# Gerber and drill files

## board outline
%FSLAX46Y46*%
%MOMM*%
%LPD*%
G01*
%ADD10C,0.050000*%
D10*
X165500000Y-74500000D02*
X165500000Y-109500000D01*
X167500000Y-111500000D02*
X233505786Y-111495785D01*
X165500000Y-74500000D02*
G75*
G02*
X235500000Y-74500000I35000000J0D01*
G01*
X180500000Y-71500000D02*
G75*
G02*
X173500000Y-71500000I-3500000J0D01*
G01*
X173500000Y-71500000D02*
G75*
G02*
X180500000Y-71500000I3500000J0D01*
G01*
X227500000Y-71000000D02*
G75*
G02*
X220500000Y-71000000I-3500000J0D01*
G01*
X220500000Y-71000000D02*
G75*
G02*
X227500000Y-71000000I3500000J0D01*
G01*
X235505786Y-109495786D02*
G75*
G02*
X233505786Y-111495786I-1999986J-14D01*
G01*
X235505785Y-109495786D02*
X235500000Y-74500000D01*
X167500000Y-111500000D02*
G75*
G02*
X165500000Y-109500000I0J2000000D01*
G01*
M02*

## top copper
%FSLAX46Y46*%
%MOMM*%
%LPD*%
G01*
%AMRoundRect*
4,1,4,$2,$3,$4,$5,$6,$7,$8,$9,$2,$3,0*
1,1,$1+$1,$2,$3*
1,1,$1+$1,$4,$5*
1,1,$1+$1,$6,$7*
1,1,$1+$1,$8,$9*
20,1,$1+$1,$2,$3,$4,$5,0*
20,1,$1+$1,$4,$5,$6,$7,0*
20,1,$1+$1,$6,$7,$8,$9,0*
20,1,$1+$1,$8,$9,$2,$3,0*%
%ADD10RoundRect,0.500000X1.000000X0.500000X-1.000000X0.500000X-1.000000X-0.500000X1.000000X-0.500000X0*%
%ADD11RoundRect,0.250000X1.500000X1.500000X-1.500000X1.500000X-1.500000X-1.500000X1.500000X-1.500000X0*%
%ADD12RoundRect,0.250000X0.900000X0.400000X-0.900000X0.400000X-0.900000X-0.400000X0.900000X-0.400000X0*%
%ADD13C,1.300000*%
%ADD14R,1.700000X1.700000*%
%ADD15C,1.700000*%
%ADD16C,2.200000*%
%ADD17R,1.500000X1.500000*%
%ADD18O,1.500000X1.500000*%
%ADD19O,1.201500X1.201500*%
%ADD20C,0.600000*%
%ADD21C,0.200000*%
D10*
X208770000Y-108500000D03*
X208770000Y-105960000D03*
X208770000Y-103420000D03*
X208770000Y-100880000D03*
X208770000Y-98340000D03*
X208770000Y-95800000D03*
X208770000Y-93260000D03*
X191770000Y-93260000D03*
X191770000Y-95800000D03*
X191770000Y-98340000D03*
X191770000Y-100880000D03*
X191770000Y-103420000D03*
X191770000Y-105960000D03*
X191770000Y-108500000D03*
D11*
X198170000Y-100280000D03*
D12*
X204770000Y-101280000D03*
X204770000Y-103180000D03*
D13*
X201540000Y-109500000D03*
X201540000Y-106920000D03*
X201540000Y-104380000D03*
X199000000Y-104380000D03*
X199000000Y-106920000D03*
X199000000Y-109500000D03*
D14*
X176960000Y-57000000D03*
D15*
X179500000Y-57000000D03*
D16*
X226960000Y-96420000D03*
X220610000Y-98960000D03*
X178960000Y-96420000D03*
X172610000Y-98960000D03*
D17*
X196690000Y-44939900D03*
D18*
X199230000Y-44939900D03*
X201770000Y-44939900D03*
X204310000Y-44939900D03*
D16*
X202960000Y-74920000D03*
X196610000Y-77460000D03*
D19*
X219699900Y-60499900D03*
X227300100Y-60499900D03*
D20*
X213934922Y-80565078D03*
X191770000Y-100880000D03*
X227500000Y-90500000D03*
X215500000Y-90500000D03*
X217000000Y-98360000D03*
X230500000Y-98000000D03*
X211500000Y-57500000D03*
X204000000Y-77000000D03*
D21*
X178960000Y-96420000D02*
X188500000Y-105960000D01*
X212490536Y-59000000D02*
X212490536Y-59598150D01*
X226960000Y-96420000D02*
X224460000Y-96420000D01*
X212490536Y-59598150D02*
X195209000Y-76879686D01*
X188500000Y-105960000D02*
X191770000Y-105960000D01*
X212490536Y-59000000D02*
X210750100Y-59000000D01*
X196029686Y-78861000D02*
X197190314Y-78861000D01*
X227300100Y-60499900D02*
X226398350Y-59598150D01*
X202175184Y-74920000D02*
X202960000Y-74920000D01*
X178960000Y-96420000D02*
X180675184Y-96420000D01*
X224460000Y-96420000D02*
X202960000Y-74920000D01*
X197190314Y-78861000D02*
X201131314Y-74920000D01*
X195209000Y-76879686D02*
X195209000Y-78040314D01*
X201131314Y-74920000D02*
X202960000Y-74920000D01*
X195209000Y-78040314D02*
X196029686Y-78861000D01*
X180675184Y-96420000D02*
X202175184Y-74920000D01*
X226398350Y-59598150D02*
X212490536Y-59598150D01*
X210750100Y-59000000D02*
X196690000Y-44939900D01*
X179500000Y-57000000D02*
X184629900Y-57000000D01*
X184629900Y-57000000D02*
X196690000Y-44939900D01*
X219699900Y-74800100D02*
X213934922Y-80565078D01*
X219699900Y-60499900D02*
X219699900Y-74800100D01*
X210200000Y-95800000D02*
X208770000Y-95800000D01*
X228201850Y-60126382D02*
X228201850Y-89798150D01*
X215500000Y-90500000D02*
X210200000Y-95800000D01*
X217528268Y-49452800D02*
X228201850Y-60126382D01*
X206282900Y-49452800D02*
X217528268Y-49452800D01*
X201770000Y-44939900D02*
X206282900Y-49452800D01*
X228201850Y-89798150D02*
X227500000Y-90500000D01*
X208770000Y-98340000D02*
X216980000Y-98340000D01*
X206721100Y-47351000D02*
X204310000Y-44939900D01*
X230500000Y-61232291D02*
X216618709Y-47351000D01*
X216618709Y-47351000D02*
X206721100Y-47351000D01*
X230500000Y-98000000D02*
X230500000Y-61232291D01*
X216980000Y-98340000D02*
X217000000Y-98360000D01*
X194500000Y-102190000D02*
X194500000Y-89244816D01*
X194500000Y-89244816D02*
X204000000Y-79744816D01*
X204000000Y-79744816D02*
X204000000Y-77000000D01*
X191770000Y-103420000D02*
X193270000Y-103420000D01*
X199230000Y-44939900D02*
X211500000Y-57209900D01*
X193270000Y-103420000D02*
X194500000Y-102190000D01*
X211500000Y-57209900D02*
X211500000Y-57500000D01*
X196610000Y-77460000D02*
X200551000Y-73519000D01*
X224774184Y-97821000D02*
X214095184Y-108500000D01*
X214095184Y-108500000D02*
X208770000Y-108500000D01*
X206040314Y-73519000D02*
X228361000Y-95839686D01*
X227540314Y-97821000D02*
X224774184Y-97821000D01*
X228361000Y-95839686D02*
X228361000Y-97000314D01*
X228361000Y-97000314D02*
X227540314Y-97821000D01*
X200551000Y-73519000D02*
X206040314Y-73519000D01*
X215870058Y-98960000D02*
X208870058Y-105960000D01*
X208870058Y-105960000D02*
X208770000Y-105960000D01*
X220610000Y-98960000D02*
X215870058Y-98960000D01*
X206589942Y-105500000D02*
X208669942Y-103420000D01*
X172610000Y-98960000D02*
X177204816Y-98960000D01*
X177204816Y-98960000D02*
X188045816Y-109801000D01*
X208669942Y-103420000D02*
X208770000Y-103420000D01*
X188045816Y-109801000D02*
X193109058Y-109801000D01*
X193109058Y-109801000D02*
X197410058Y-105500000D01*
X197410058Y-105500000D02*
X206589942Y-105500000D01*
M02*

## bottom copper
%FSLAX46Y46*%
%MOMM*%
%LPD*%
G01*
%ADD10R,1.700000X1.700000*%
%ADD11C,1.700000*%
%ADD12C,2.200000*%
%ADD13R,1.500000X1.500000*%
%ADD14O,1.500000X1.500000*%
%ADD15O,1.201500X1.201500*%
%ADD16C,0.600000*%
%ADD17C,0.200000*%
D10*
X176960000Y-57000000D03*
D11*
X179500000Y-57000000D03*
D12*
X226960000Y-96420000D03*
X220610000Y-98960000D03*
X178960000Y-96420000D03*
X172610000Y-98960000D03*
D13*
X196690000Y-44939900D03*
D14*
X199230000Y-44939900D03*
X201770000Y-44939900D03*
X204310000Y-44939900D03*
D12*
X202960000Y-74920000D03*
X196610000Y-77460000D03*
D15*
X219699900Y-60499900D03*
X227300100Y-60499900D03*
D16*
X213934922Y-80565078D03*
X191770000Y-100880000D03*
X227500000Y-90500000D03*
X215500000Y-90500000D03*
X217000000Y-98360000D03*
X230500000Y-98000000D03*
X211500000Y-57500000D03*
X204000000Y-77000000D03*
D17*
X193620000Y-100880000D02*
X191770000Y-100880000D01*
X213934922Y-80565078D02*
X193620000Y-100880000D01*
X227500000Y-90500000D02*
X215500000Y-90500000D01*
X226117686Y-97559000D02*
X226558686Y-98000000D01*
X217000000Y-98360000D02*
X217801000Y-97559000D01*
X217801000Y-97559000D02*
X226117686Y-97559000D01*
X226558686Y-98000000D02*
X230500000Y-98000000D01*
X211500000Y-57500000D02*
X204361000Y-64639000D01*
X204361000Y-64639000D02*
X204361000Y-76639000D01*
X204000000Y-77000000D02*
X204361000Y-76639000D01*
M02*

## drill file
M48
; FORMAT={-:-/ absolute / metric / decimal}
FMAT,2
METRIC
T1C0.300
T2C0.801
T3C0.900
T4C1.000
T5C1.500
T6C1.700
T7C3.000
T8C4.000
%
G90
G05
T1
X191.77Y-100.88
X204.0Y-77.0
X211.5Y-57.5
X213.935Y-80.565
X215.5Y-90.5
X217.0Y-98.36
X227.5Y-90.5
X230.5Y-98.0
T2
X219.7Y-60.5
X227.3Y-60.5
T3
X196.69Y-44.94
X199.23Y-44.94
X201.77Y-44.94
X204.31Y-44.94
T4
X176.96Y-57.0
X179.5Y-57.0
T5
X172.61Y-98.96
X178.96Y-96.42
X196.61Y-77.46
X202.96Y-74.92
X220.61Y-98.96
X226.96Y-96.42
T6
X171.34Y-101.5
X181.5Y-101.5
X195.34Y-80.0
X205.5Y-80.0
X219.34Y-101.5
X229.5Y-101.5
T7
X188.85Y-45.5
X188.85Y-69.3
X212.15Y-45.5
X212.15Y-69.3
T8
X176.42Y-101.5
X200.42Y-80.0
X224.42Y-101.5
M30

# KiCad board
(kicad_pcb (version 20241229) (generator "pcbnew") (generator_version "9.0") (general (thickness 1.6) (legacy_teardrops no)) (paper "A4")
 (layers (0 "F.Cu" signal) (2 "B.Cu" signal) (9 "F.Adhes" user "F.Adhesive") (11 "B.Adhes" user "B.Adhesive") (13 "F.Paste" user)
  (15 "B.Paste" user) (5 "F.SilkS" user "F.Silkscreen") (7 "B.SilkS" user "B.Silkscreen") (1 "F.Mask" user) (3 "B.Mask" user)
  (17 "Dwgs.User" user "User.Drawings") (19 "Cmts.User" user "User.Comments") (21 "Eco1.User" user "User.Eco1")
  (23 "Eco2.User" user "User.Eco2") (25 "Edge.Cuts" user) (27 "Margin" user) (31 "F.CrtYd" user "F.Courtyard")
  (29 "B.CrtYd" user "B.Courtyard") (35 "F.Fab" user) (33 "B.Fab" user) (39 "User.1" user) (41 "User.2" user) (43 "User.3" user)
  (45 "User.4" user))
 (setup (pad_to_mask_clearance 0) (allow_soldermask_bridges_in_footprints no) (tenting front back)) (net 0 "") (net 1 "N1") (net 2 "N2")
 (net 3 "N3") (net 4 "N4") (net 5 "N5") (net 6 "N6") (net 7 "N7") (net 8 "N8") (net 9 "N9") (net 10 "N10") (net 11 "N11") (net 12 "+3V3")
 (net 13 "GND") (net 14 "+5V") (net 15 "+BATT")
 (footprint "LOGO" (layer "F.Cu") (at 225.5 79.5 -90)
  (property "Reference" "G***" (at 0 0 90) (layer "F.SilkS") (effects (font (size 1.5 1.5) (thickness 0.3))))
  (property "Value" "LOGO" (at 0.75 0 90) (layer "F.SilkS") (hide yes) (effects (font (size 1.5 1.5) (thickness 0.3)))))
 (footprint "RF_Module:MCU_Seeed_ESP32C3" (layer "F.Cu") (at 200.27 100.88 180)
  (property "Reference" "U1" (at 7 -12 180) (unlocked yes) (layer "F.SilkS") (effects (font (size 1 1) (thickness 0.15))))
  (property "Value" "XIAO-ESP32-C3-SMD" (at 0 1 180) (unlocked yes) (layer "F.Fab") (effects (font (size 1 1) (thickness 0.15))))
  (pad "" smd roundrect (at 1.1 -0.4 180) (size 1.5 1.5) (layers "F.Paste") (roundrect_rratio 0.1666666667))
  (pad "" smd roundrect (at 1.1 1.6 180) (size 1.5 1.5) (layers "F.Paste") (roundrect_rratio 0.1666666667))
  (pad "" smd roundrect (at 3.1 -0.4 180) (size 1.5 1.5) (layers "F.Paste") (roundrect_rratio 0.1666666667))
  (pad "" smd roundrect (at 3.1 1.6 180) (size 1.5 1.5) (layers "F.Paste") (roundrect_rratio 0.1666666667))
  (pad "1" smd roundrect (at -8.5 -7.62 180) (size 3 2) (layers "F.Cu" "F.Mask" "F.Paste") (roundrect_rratio 0.25) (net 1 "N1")
   (thermal_bridge_angle 45))
  (pad "2" smd roundrect (at -8.5 -5.08 180) (size 3 2) (layers "F.Cu" "F.Mask" "F.Paste") (roundrect_rratio 0.25) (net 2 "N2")
   (thermal_bridge_angle 45))
  (pad "3" smd roundrect (at -8.5 -2.54 180) (size 3 2) (layers "F.Cu" "F.Mask" "F.Paste") (roundrect_rratio 0.25) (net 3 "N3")
   (thermal_bridge_angle 45))
  (pad "4" smd roundrect (at -8.5 0 180) (size 3 2) (layers "F.Cu" "F.Mask" "F.Paste") (roundrect_rratio 0.25) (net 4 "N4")
   (thermal_bridge_angle 45))
  (pad "5" smd roundrect (at -8.5 2.54 180) (size 3 2) (layers "F.Cu" "F.Mask" "F.Paste") (roundrect_rratio 0.25) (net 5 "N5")
   (thermal_bridge_angle 45))
  (pad "6" smd roundrect (at -8.5 5.08 180) (size 3 2) (layers "F.Cu" "F.Mask" "F.Paste") (roundrect_rratio 0.25) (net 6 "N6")
   (thermal_bridge_angle 45))
  (pad "7" smd roundrect (at -8.5 7.62 180) (size 3 2) (layers "F.Cu" "F.Mask" "F.Paste") (roundrect_rratio 0.25) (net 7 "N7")
   (thermal_bridge_angle 45))
  (pad "8" smd roundrect (at 8.5 7.62 180) (size 3 2) (layers "F.Cu" "F.Mask" "F.Paste") (roundrect_rratio 0.25) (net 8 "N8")
   (thermal_bridge_angle 45))
  (pad "9" smd roundrect (at 8.5 5.08 180) (size 3 2) (layers "F.Cu" "F.Mask" "F.Paste") (roundrect_rratio 0.25) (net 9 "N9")
   (thermal_bridge_angle 45))
  (pad "10" smd roundrect (at 8.5 2.54 180) (size 3 2) (layers "F.Cu" "F.Mask" "F.Paste") (roundrect_rratio 0.25) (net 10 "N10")
   (thermal_bridge_angle 45))
  (pad "11" smd roundrect (at 8.5 0 180) (size 3 2) (layers "F.Cu" "F.Mask" "F.Paste") (roundrect_rratio 0.25) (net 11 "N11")
   (thermal_bridge_angle 45))
  (pad "12" smd roundrect (at 8.5 -2.54 180) (size 3 2) (layers "F.Cu" "F.Mask" "F.Paste") (roundrect_rratio 0.25) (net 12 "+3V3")
   (thermal_bridge_angle 45))
  (pad "13" smd roundrect (at 8.5 -5.08 180) (size 3 2) (layers "F.Cu" "F.Mask" "F.Paste") (roundrect_rratio 0.25) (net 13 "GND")
   (thermal_bridge_angle 45))
  (pad "14" smd roundrect (at 8.5 -7.62 180) (size 3 2) (layers "F.Cu" "F.Mask" "F.Paste") (roundrect_rratio 0.25) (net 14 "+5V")
   (thermal_bridge_angle 45))
  (pad "15" smd roundrect (at 2.1 0.6 180) (size 3.5 3.5) (layers "F.Cu" "F.Mask") (roundrect_rratio 0.07142857143))
  (pad "16" smd roundrect (at -4.5 -0.4 180) (size 2.3 1.3) (layers "F.Cu" "F.Mask" "F.Paste") (roundrect_rratio 0.1923076923))
  (pad "17" smd roundrect (at -4.5 -2.3 180) (size 2.3 1.3) (layers "F.Cu" "F.Mask" "F.Paste") (roundrect_rratio 0.1923076923))
  (pad "18" smd circle (at -1.27 -8.62 180) (size 1.3 1.3) (layers "F.Cu" "F.Mask" "F.Paste"))
  (pad "19" smd circle (at -1.27 -6.04 180) (size 1.3 1.3) (layers "F.Cu" "F.Mask" "F.Paste"))
  (pad "20" smd circle (at -1.27 -3.5 180) (size 1.3 1.3) (layers "F.Cu" "F.Mask" "F.Paste"))
  (pad "21" smd circle (at 1.27 -3.5 180) (size 1.3 1.3) (layers "F.Cu" "F.Mask" "F.Paste"))
  (pad "22" smd circle (at 1.27 -6.04 180) (size 1.3 1.3) (layers "F.Cu" "F.Mask" "F.Paste"))
  (pad "23" smd circle (at 1.27 -8.62 180) (size 1.3 1.3) (layers "F.Cu" "F.Mask" "F.Paste")))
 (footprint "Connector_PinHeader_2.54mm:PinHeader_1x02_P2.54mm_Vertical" (layer "F.Cu") (at 176.96 57 90)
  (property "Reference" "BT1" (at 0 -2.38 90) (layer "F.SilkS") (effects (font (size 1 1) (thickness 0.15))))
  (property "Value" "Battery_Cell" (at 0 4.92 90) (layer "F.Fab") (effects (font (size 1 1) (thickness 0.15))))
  (pad "1" thru_hole rect (at 0 0 90) (size 1.7 1.7) (drill 1) (layers "*.Cu" "*.Mask") (remove_unused_layers no) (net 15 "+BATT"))
  (pad "2" thru_hole circle (at 0 2.54 90) (size 1.7 1.7) (drill 1) (layers "*.Cu" "*.Mask") (remove_unused_layers no) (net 13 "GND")))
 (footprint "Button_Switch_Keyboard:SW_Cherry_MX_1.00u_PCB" (layer "F.Cu") (at 226.96 96.42)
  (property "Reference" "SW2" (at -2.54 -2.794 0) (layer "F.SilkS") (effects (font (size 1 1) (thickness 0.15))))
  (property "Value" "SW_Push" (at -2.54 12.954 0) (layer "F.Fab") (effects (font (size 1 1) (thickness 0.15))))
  (pad "" np_thru_hole circle (at -7.62 5.08) (size 1.7 1.7) (drill 1.7) (layers "*.Cu" "*.Mask"))
  (pad "" np_thru_hole circle (at -2.54 5.08) (size 4 4) (drill 4) (layers "*.Cu" "*.Mask"))
  (pad "" np_thru_hole circle (at 2.54 5.08) (size 1.7 1.7) (drill 1.7) (layers "*.Cu" "*.Mask"))
  (pad "1" thru_hole circle (at 0 0) (size 2.2 2.2) (drill 1.5) (layers "*.Cu" "*.Mask") (remove_unused_layers no) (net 13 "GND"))
  (pad "2" thru_hole circle (at -6.35 2.54) (size 2.2 2.2) (drill 1.5) (layers "*.Cu" "*.Mask") (remove_unused_layers no) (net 2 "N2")))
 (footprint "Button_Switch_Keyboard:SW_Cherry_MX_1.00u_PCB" (layer "F.Cu") (at 178.96 96.42)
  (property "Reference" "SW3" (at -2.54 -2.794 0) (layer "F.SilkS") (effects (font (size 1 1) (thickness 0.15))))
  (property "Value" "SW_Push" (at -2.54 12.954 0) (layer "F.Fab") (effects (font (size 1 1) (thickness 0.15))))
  (pad "" np_thru_hole circle (at -7.62 5.08) (size 1.7 1.7) (drill 1.7) (layers "*.Cu" "*.Mask"))
  (pad "" np_thru_hole circle (at -2.54 5.08) (size 4 4) (drill 4) (layers "*.Cu" "*.Mask"))
  (pad "" np_thru_hole circle (at 2.54 5.08) (size 1.7 1.7) (drill 1.7) (layers "*.Cu" "*.Mask"))
  (pad "1" thru_hole circle (at 0 0) (size 2.2 2.2) (drill 1.5) (layers "*.Cu" "*.Mask") (remove_unused_layers no) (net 13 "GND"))
  (pad "2" thru_hole circle (at -6.35 2.54) (size 2.2 2.2) (drill 1.5) (layers "*.Cu" "*.Mask") (remove_unused_layers no) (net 3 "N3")))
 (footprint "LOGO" (layer "F.Cu") (at 177.5 78)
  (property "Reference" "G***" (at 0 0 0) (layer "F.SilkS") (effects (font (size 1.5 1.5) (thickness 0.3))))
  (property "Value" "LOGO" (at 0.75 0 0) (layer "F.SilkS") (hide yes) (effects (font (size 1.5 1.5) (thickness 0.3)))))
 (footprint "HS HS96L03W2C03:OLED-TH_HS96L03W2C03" (layer "F.Cu") (at 200.5 44.9399)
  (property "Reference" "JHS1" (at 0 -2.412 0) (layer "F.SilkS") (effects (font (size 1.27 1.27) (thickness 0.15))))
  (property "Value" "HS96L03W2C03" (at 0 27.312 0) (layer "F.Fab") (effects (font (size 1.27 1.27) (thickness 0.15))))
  (pad "" np_thru_hole circle (at -11.65 0.5601) (size 3 3) (drill 3) (layers "*.Cu" "*.Mask"))
  (pad "" np_thru_hole circle (at -11.65 24.3599) (size 3 3) (drill 3) (layers "*.Cu" "*.Mask"))
  (pad "" np_thru_hole circle (at 11.65 0.5601) (size 3 3) (drill 3) (layers "*.Cu" "*.Mask"))
  (pad "" np_thru_hole circle (at 11.65 24.3599) (size 3 3) (drill 3) (layers "*.Cu" "*.Mask"))
  (pad "1" thru_hole rect (at -3.81 0) (size 1.5 1.5) (drill 0.9) (layers "*.Cu" "*.Mask") (remove_unused_layers no) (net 13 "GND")
   (solder_mask_margin 0.05) (solder_paste_margin 0) (thermal_bridge_angle 0))
  (pad "2" thru_hole oval (at -1.27 0) (size 1.5 1.5) (drill 0.9) (layers "*.Cu" "*.Mask") (remove_unused_layers no) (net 12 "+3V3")
   (solder_mask_margin 0.05) (solder_paste_margin 0) (thermal_bridge_angle 0))
  (pad "3" thru_hole oval (at 1.27 0) (size 1.5 1.5) (drill 0.9) (layers "*.Cu" "*.Mask") (remove_unused_layers no) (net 6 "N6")
   (solder_mask_margin 0.05) (solder_paste_margin 0) (thermal_bridge_angle 0))
  (pad "4" thru_hole oval (at 3.81 0) (size 1.5 1.5) (drill 0.9) (layers "*.Cu" "*.Mask") (remove_unused_layers no) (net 5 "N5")
   (solder_mask_margin 0.05) (solder_paste_margin 0) (thermal_bridge_angle 0))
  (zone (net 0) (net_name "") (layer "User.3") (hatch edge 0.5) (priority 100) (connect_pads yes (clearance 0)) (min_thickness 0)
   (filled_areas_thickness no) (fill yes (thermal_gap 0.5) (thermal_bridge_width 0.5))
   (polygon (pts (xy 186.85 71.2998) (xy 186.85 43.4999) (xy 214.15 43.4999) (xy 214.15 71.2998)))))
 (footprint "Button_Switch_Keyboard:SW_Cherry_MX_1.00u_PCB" (layer "F.Cu") (at 202.96 74.92)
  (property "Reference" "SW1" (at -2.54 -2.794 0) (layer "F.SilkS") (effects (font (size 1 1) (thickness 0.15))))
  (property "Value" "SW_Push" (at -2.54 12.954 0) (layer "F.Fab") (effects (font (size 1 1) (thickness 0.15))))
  (pad "" np_thru_hole circle (at -7.62 5.08) (size 1.7 1.7) (drill 1.7) (layers "*.Cu" "*.Mask"))
  (pad "" np_thru_hole circle (at -2.54 5.08) (size 4 4) (drill 4) (layers "*.Cu" "*.Mask"))
  (pad "" np_thru_hole circle (at 2.54 5.08) (size 1.7 1.7) (drill 1.7) (layers "*.Cu" "*.Mask"))
  (pad "1" thru_hole circle (at 0 0) (size 2.2 2.2) (drill 1.5) (layers "*.Cu" "*.Mask") (remove_unused_layers no) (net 13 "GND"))
  (pad "2" thru_hole circle (at -6.35 2.54) (size 2.2 2.2) (drill 1.5) (layers "*.Cu" "*.Mask") (remove_unused_layers no) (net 1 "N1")))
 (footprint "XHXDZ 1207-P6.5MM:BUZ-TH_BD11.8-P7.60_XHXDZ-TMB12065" (layer "F.Cu") (at 223.5 60.5 90)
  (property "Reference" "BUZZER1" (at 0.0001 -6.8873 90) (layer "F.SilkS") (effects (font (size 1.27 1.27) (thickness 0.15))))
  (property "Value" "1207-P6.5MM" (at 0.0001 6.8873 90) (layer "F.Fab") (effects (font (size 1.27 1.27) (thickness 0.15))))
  (pad "1" thru_hole oval (at 0.0001 -3.8001) (size 1.2015 1.2015) (drill 0.801) (layers "*.Cu" "*.Mask") (remove_unused_layers no)
   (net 11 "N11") (solder_mask_margin 0.0508) (solder_paste_margin 0) (thermal_bridge_angle 0))
  (pad "2" thru_hole oval (at 0.0001 3.8001 180) (size 1.2015 1.2015) (drill 0.801) (layers "*.Cu" "*.Mask") (remove_unused_layers no)
   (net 13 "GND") (solder_mask_margin 0.0508) (solder_paste_margin 0) (thermal_bridge_angle 0))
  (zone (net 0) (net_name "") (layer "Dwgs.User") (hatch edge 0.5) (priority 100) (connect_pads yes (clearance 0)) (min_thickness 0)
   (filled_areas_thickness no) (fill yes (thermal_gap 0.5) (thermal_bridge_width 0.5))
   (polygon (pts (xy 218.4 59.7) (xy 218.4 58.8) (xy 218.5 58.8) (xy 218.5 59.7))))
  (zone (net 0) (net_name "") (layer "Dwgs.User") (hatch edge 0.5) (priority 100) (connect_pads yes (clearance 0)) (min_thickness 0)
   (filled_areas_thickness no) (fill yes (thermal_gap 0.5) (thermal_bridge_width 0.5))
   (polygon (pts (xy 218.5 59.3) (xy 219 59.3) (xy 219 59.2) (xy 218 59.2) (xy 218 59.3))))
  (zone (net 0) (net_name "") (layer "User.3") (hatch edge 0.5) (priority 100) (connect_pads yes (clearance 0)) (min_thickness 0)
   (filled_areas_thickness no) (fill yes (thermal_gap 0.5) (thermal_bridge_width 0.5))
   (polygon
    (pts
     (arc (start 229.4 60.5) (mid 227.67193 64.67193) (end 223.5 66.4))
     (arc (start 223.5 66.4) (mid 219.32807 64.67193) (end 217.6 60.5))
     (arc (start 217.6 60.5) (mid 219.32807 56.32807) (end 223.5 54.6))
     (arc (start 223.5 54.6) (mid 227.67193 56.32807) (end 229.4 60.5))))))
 (gr_line (start 165.5 74.5) (end 165.5 109.5) (stroke (width 0.05) (type default)) (layer "Edge.Cuts"))
 (gr_line (start 167.5 111.5) (end 233.505786 111.495785) (stroke (width 0.05) (type default)) (layer "Edge.Cuts"))
 (gr_arc (start 165.5 74.5) (mid 200.5 39.5) (end 235.5 74.5) (stroke (width 0.05) (type default)) (layer "Edge.Cuts"))
 (gr_circle (center 177 71.5) (end 180.5 71.5) (stroke (width 0.05) (type default)) (fill no) (layer "Edge.Cuts"))
 (gr_circle (center 224 71) (end 227.5 71) (stroke (width 0.05) (type default)) (fill no) (layer "Edge.Cuts"))
 (gr_arc (start 235.505786 109.495786) (mid 234.92 110.91) (end 233.505786 111.495786) (stroke (width 0.05) (type default))
  (layer "Edge.Cuts"))
 (gr_line (start 235.505785 109.495786) (end 235.5 74.5) (stroke (width 0.05) (type default)) (layer "Edge.Cuts"))
 (gr_arc (start 167.5 111.5) (mid 166.085786 110.914214) (end 165.5 109.5) (stroke (width 0.05) (type default)) (layer "Edge.Cuts"))
 (segment (start 178.96 96.42) (end 188.5 105.96) (width 0.2) (layer "F.Cu") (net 13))
 (segment (start 212.490536 59) (end 212.490536 59.59815) (width 0.2) (layer "F.Cu") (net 13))
 (segment (start 226.96 96.42) (end 224.46 96.42) (width 0.2) (layer "F.Cu") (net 13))
 (segment (start 212.490536 59.59815) (end 195.209 76.879686) (width 0.2) (layer "F.Cu") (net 13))
 (segment (start 188.5 105.96) (end 191.77 105.96) (width 0.2) (layer "F.Cu") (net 13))
 (segment (start 212.490536 59) (end 210.7501 59) (width 0.2) (layer "F.Cu") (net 13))
 (segment (start 196.029686 78.861) (end 197.190314 78.861) (width 0.2) (layer "F.Cu") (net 13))
 (segment (start 227.3001 60.4999) (end 226.39835 59.59815) (width 0.2) (layer "F.Cu") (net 13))
 (segment (start 202.175184 74.92) (end 202.96 74.92) (width 0.2) (layer "F.Cu") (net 13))
 (segment (start 178.96 96.42) (end 180.675184 96.42) (width 0.2) (layer "F.Cu") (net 13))
 (segment (start 224.46 96.42) (end 202.96 74.92) (width 0.2) (layer "F.Cu") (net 13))
 (segment (start 197.190314 78.861) (end 201.131314 74.92) (width 0.2) (layer "F.Cu") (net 13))
 (segment (start 195.209 76.879686) (end 195.209 78.040314) (width 0.2) (layer "F.Cu") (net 13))
 (segment (start 201.131314 74.92) (end 202.96 74.92) (width 0.2) (layer "F.Cu") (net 13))
 (segment (start 195.209 78.040314) (end 196.029686 78.861) (width 0.2) (layer "F.Cu") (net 13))
 (segment (start 180.675184 96.42) (end 202.175184 74.92) (width 0.2) (layer "F.Cu") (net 13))
 (segment (start 226.39835 59.59815) (end 212.490536 59.59815) (width 0.2) (layer "F.Cu") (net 13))
 (segment (start 210.7501 59) (end 196.69 44.9399) (width 0.2) (layer "F.Cu") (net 13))
 (segment (start 179.5 57) (end 184.6299 57) (width 0.2) (layer "F.Cu") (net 13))
 (segment (start 184.6299 57) (end 196.69 44.9399) (width 0.2) (layer "F.Cu") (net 13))
 (segment (start 219.6999 74.8001) (end 213.934922 80.565078) (width 0.2) (layer "F.Cu") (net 11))
 (segment (start 219.6999 60.4999) (end 219.6999 74.8001) (width 0.2) (layer "F.Cu") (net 11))
 (via (at 213.934922 80.565078) (size 0.6) (drill 0.3) (layers "F.Cu" "B.Cu") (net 11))
 (via (at 191.77 100.88) (size 0.6) (drill 0.3) (layers "F.Cu" "B.Cu") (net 11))
 (segment (start 193.62 100.88) (end 191.77 100.88) (width 0.2) (layer "B.Cu") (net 11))
 (segment (start 213.934922 80.565078) (end 193.62 100.88) (width 0.2) (layer "B.Cu") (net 11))
 (segment (start 210.2 95.8) (end 208.77 95.8) (width 0.2) (layer "F.Cu") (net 6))
 (segment (start 228.20185 60.126382) (end 228.20185 89.79815) (width 0.2) (layer "F.Cu") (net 6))
 (segment (start 215.5 90.5) (end 210.2 95.8) (width 0.2) (layer "F.Cu") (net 6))
 (segment (start 217.528268 49.4528) (end 228.20185 60.126382) (width 0.2) (layer "F.Cu") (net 6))
 (segment (start 206.2829 49.4528) (end 217.528268 49.4528) (width 0.2) (layer "F.Cu") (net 6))
 (segment (start 201.77 44.9399) (end 206.2829 49.4528) (width 0.2) (layer "F.Cu") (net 6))
 (segment (start 228.20185 89.79815) (end 227.5 90.5) (width 0.2) (layer "F.Cu") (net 6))
 (via (at 227.5 90.5) (size 0.6) (drill 0.3) (layers "F.Cu" "B.Cu") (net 6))
 (via (at 215.5 90.5) (size 0.6) (drill 0.3) (layers "F.Cu" "B.Cu") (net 6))
 (segment (start 227.5 90.5) (end 215.5 90.5) (width 0.2) (layer "B.Cu") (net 6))
 (segment (start 208.77 98.34) (end 216.98 98.34) (width 0.2) (layer "F.Cu") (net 5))
 (segment (start 206.7211 47.351) (end 204.31 44.9399) (width 0.2) (layer "F.Cu") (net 5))
 (segment (start 230.5 61.232291) (end 216.618709 47.351) (width 0.2) (layer "F.Cu") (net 5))
 (segment (start 216.618709 47.351) (end 206.7211 47.351) (width 0.2) (layer "F.Cu") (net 5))
 (segment (start 230.5 98) (end 230.5 61.232291) (width 0.2) (layer "F.Cu") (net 5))
 (segment (start 216.98 98.34) (end 217 98.36) (width 0.2) (layer "F.Cu") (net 5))
 (via (at 217 98.36) (size 0.6) (drill 0.3) (layers "F.Cu" "B.Cu") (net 5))
 (via (at 230.5 98) (size 0.6) (drill 0.3) (layers "F.Cu" "B.Cu") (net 5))
 (segment (start 226.117686 97.559) (end 226.558686 98) (width 0.2) (layer "B.Cu") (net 5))
 (segment (start 217 98.36) (end 217.801 97.559) (width 0.2) (layer "B.Cu") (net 5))
 (segment (start 217.801 97.559) (end 226.117686 97.559) (width 0.2) (layer "B.Cu") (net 5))
 (segment (start 226.558686 98) (end 230.5 98) (width 0.2) (layer "B.Cu") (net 5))
 (segment (start 194.5 102.19) (end 194.5 89.244816) (width 0.2) (layer "F.Cu") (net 12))
 (segment (start 194.5 89.244816) (end 204 79.744816) (width 0.2) (layer "F.Cu") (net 12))
 (segment (start 204 79.744816) (end 204 77) (width 0.2) (layer "F.Cu") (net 12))
 (segment (start 191.77 103.42) (end 193.27 103.42) (width 0.2) (layer "F.Cu") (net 12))
 (segment (start 199.23 44.9399) (end 211.5 57.2099) (width 0.2) (layer "F.Cu") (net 12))
 (segment (start 193.27 103.42) (end 194.5 102.19) (width 0.2) (layer "F.Cu") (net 12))
 (segment (start 211.5 57.2099) (end 211.5 57.5) (width 0.2) (layer "F.Cu") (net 12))
 (via (at 211.5 57.5) (size 0.6) (drill 0.3) (layers "F.Cu" "B.Cu") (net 12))
 (via (at 204 77) (size 0.6) (drill 0.3) (layers "F.Cu" "B.Cu") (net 12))
 (segment (start 211.5 57.5) (end 204.361 64.639) (width 0.2) (layer "B.Cu") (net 12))
 (segment (start 204.361 64.639) (end 204.361 76.639) (width 0.2) (layer "B.Cu") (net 12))
 (segment (start 204 77) (end 204.361 76.639) (width 0.2) (layer "B.Cu") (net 12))
 (segment (start 196.61 77.46) (end 200.551 73.519) (width 0.2) (layer "F.Cu") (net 1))
 (segment (start 224.774184 97.821) (end 214.095184 108.5) (width 0.2) (layer "F.Cu") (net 1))
 (segment (start 214.095184 108.5) (end 208.77 108.5) (width 0.2) (layer "F.Cu") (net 1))
 (segment (start 206.040314 73.519) (end 228.361 95.839686) (width 0.2) (layer "F.Cu") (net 1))
 (segment (start 227.540314 97.821) (end 224.774184 97.821) (width 0.2) (layer "F.Cu") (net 1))
 (segment (start 228.361 95.839686) (end 228.361 97.000314) (width 0.2) (layer "F.Cu") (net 1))
 (segment (start 228.361 97.000314) (end 227.540314 97.821) (width 0.2) (layer "F.Cu") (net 1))
 (segment (start 200.551 73.519) (end 206.040314 73.519) (width 0.2) (layer "F.Cu") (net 1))
 (segment (start 215.870058 98.96) (end 208.870058 105.96) (width 0.2) (layer "F.Cu") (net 2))
 (segment (start 208.870058 105.96) (end 208.77 105.96) (width 0.2) (layer "F.Cu") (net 2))
 (segment (start 220.61 98.96) (end 215.870058 98.96) (width 0.2) (layer "F.Cu") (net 2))
 (segment (start 206.589942 105.5) (end 208.669942 103.42) (width 0.2) (layer "F.Cu") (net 3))
 (segment (start 172.61 98.96) (end 177.204816 98.96) (width 0.2) (layer "F.Cu") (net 3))
 (segment (start 177.204816 98.96) (end 188.045816 109.801) (width 0.2) (layer "F.Cu") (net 3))
 (segment (start 208.669942 103.42) (end 208.77 103.42) (width 0.2) (layer "F.Cu") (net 3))
 (segment (start 188.045816 109.801) (end 193.109058 109.801) (width 0.2) (layer "F.Cu") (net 3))
 (segment (start 193.109058 109.801) (end 197.410058 105.5) (width 0.2) (layer "F.Cu") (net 3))
 (segment (start 197.410058 105.5) (end 206.589942 105.5) (width 0.2) (layer "F.Cu") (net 3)))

